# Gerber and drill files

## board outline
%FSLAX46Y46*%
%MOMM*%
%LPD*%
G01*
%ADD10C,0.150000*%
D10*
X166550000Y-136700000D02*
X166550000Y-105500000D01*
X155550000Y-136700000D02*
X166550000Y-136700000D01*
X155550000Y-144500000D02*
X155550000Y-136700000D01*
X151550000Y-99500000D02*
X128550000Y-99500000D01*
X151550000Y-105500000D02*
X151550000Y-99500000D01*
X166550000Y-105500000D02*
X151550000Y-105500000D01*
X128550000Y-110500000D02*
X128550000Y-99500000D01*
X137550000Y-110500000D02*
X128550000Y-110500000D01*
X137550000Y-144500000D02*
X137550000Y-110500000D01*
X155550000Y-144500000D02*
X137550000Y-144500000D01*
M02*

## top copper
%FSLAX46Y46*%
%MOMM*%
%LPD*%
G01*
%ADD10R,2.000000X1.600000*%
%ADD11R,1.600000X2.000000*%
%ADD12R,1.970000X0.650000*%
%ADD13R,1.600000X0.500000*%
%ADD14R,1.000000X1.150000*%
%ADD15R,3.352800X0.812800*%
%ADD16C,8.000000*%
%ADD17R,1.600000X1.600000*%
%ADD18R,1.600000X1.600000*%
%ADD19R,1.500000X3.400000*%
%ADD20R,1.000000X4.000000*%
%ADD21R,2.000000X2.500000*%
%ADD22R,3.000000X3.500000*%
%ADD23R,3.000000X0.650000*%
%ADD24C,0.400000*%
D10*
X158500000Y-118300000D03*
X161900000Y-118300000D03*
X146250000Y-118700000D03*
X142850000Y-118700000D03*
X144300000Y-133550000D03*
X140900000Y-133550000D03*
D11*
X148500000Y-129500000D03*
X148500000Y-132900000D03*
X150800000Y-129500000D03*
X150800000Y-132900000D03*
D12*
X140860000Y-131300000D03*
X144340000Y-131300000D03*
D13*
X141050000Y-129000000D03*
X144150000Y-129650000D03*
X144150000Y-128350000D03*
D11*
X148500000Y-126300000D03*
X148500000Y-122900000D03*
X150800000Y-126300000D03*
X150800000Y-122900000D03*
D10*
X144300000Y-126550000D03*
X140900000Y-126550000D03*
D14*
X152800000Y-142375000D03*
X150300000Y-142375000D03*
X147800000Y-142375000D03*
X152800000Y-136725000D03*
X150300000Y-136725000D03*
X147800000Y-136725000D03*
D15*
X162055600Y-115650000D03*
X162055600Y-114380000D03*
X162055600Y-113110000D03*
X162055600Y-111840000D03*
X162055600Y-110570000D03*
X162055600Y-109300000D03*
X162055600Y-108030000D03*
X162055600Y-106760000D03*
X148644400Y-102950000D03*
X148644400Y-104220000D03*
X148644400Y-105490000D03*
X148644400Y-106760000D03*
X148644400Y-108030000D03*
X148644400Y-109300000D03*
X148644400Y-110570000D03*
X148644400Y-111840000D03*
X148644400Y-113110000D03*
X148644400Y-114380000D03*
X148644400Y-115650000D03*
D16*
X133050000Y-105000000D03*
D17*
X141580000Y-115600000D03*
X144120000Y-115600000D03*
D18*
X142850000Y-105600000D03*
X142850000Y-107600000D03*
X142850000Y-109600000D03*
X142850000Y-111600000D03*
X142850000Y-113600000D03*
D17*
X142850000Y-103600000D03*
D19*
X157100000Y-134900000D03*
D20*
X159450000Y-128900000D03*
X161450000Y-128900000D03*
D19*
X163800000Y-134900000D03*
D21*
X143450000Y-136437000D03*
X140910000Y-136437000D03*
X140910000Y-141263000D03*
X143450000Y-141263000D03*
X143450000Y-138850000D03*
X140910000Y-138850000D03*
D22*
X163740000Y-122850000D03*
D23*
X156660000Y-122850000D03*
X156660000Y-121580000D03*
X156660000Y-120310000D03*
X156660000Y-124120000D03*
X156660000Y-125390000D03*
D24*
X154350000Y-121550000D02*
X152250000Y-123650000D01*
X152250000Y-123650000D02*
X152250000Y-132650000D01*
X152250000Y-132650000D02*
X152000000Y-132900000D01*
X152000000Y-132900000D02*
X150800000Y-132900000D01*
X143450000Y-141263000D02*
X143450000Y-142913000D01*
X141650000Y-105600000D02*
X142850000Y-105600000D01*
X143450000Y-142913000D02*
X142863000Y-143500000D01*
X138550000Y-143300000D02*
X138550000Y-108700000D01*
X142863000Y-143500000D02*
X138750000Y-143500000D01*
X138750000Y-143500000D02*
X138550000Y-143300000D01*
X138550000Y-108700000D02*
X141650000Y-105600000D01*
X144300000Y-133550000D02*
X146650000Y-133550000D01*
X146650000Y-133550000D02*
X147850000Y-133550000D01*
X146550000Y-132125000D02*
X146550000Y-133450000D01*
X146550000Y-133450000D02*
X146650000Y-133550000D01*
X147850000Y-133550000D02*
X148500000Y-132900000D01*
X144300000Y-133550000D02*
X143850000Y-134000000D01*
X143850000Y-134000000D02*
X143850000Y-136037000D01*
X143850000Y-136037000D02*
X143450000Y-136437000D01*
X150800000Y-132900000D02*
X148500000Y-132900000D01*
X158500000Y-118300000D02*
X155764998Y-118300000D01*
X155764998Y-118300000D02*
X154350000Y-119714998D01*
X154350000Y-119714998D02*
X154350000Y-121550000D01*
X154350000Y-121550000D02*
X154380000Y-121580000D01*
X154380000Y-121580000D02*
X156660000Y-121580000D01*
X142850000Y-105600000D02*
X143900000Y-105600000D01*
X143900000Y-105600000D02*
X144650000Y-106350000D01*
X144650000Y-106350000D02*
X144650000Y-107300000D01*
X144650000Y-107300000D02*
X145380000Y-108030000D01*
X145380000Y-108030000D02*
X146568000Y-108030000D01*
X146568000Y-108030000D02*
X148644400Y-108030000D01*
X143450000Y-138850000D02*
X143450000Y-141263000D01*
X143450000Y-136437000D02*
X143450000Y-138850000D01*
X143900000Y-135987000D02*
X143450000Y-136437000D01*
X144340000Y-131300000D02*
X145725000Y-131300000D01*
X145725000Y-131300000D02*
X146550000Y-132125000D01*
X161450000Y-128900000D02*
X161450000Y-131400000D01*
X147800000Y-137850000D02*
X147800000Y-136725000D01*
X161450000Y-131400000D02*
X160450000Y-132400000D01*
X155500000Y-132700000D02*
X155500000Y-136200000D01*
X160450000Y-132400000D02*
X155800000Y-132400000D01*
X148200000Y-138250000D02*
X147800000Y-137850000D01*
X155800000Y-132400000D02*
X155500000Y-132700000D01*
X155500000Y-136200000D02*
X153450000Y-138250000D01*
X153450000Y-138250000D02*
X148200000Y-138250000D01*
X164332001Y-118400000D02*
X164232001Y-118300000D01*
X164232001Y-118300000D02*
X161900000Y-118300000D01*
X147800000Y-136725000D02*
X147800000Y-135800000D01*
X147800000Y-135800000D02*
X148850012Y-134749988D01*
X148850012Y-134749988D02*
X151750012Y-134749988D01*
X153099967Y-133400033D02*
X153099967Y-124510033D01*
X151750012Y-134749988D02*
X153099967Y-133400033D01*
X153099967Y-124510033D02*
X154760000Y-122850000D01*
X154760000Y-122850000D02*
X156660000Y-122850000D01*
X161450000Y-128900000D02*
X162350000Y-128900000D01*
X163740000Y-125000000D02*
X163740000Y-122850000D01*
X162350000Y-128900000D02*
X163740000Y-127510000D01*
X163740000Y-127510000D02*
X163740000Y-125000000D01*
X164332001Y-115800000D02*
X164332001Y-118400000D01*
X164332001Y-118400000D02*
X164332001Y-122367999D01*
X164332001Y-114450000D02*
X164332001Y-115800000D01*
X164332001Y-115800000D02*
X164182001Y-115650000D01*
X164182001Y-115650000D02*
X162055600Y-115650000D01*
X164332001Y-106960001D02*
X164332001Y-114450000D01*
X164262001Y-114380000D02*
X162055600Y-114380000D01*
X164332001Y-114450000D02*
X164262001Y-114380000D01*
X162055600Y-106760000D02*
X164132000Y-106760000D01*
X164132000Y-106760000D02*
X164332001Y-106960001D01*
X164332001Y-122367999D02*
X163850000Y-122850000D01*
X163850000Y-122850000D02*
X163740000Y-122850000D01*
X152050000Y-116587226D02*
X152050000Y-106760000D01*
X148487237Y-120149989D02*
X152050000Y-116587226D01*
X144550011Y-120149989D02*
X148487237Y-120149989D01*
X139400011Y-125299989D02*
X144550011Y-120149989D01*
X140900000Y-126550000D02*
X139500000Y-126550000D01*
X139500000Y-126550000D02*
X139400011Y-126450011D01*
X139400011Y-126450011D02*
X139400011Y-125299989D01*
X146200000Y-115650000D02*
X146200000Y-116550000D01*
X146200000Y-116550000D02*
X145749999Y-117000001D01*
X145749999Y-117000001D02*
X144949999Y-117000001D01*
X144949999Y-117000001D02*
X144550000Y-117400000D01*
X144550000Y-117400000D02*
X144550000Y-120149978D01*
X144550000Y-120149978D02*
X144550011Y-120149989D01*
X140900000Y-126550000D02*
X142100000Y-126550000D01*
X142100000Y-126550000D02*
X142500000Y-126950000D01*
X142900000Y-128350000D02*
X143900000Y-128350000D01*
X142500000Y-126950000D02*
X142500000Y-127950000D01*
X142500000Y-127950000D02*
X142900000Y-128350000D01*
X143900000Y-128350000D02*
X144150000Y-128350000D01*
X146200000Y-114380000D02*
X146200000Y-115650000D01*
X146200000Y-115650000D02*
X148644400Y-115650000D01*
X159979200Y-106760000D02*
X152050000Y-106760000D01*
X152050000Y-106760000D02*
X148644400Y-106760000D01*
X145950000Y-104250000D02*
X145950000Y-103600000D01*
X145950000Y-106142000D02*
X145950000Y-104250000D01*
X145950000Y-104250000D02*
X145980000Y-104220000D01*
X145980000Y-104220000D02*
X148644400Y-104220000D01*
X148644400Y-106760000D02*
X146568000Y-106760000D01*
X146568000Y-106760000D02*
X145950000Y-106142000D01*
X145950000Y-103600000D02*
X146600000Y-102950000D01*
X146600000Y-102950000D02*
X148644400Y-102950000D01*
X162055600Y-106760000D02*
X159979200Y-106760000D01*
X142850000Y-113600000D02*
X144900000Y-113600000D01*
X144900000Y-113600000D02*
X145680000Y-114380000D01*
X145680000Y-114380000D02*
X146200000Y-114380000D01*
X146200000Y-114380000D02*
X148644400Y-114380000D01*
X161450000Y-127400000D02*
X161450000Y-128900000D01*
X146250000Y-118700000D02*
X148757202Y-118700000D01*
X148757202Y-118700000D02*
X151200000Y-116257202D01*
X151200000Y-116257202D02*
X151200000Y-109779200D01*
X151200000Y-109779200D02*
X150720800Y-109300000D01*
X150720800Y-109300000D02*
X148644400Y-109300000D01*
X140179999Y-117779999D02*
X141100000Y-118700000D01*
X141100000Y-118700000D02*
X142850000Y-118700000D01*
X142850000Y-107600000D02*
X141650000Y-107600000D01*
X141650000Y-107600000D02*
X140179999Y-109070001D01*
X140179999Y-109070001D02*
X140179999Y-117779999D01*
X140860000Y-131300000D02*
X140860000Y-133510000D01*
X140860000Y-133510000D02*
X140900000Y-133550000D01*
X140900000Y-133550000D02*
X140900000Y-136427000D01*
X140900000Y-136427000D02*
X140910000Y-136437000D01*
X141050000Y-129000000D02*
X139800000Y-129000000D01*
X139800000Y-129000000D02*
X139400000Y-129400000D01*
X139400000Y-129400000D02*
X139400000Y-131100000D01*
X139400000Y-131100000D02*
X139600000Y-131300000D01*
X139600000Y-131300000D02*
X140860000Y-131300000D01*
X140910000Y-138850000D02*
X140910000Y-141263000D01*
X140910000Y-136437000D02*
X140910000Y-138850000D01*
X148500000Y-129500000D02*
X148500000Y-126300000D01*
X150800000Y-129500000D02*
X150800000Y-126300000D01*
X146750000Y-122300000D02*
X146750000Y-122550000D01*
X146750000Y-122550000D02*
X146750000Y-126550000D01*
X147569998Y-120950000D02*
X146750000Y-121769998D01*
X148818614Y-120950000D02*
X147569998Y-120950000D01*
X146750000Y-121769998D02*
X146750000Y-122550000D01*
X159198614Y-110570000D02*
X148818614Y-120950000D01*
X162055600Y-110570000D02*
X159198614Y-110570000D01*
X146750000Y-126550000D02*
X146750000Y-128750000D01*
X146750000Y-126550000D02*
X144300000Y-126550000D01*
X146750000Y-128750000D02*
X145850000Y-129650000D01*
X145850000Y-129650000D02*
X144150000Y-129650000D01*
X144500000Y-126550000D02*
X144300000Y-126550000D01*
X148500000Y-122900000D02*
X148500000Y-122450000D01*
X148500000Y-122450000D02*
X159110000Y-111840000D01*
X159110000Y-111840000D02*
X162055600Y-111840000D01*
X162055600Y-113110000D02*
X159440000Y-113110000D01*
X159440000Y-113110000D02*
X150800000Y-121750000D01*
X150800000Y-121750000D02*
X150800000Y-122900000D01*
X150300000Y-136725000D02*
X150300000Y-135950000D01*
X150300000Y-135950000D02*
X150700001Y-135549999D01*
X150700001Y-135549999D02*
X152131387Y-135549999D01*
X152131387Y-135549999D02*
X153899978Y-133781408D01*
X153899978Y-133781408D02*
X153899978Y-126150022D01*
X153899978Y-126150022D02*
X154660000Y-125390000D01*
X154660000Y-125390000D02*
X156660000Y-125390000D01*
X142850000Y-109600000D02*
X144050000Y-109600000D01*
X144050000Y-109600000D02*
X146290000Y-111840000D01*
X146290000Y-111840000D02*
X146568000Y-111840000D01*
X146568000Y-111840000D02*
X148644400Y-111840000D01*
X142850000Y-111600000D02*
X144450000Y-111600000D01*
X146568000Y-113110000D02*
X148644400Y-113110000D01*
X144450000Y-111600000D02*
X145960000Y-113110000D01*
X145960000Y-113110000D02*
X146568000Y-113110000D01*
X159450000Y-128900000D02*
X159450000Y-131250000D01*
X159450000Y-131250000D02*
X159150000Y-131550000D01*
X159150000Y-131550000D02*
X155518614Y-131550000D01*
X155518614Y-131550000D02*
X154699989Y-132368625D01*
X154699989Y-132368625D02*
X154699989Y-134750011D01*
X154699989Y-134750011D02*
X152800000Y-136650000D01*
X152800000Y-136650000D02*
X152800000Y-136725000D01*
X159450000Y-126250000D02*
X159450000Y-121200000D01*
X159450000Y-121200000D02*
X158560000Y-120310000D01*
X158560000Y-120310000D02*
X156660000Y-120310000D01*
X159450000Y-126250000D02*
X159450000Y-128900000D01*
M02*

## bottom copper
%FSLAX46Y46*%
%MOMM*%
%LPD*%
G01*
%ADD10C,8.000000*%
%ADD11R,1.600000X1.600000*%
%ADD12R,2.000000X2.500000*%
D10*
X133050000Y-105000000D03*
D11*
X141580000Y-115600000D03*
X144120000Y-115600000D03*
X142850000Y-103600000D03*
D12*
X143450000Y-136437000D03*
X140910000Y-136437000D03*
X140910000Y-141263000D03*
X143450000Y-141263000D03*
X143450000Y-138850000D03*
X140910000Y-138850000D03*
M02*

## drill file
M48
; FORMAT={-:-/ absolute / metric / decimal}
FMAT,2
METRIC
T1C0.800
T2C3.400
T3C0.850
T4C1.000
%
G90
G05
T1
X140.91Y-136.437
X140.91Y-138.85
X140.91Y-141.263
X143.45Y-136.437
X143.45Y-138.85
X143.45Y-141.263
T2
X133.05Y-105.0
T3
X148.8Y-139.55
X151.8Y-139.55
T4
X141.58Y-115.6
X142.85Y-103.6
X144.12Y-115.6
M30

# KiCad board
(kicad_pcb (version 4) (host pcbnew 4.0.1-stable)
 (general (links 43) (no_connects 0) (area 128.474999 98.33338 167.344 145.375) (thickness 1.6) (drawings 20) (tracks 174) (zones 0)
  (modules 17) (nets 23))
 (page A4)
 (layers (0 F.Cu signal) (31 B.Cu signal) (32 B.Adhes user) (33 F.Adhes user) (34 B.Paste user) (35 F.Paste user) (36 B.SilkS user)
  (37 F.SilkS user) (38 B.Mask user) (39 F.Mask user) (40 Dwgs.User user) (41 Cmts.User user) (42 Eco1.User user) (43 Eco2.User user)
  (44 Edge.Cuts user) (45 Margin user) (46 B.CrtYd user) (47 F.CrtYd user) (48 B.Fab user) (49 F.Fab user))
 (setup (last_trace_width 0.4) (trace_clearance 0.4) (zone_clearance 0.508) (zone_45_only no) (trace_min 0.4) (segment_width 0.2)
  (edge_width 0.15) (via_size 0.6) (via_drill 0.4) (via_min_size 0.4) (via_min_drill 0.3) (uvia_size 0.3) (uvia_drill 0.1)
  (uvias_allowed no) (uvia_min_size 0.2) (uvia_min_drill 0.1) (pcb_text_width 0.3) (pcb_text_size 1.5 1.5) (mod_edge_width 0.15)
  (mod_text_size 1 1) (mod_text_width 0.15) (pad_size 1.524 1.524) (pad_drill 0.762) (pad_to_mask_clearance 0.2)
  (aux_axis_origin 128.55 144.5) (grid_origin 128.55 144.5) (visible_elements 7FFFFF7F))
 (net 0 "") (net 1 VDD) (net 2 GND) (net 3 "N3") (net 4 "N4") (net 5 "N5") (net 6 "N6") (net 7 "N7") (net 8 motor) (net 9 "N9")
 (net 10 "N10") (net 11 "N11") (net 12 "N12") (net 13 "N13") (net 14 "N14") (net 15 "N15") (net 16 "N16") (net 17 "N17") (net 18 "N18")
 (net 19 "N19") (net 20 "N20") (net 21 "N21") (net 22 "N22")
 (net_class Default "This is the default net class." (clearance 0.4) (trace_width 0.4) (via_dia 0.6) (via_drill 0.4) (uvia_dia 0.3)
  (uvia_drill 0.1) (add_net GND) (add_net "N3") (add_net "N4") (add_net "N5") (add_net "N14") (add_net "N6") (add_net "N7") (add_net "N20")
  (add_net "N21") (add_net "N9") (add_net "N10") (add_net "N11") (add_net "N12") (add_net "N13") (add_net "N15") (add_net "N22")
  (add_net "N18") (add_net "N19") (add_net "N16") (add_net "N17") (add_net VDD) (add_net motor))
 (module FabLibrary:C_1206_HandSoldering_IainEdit (layer F.Cu) (at 160.2 118.3)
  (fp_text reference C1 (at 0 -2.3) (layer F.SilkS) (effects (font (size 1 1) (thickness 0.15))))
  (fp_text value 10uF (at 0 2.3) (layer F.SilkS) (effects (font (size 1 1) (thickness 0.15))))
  (pad 1 smd rect (at -1.7 0) (size 2 1.6) (layers F.Cu F.Paste F.Mask) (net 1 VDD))
  (pad 2 smd rect (at 1.7 0) (size 2 1.6) (layers F.Cu F.Paste F.Mask) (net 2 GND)))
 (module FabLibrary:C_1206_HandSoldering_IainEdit (layer F.Cu) (at 144.55 118.7 180)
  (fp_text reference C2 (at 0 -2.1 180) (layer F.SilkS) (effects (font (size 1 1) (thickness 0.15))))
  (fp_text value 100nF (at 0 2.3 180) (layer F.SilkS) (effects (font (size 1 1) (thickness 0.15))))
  (pad 1 smd rect (at -1.7 0 180) (size 2 1.6) (layers F.Cu F.Paste F.Mask) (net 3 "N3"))
  (pad 2 smd rect (at 1.7 0 180) (size 2 1.6) (layers F.Cu F.Paste F.Mask) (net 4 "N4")))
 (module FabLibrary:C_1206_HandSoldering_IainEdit (layer F.Cu) (at 142.6 133.55 180)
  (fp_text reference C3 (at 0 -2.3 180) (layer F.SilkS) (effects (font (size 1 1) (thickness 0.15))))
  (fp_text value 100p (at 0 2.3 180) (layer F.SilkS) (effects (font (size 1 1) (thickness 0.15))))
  (pad 1 smd rect (at -1.7 0 180) (size 2 1.6) (layers F.Cu F.Paste F.Mask) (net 1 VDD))
  (pad 2 smd rect (at 1.7 0 180) (size 2 1.6) (layers F.Cu F.Paste F.Mask) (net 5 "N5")))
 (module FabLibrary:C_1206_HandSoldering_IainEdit (layer F.Cu) (at 148.5 131.2 270)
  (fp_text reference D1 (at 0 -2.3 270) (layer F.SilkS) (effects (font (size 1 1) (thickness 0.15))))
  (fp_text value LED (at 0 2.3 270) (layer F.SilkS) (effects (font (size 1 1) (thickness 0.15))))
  (pad 1 smd rect (at -1.7 0 270) (size 2 1.6) (layers F.Cu F.Paste F.Mask) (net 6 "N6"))
  (pad 2 smd rect (at 1.7 0 270) (size 2 1.6) (layers F.Cu F.Paste F.Mask) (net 1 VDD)))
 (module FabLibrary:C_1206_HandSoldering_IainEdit (layer F.Cu) (at 150.8 131.2 270)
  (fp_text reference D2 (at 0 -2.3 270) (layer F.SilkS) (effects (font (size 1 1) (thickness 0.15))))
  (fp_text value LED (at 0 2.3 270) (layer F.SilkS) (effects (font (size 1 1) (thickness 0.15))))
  (pad 1 smd rect (at -1.7 0 270) (size 2 1.6) (layers F.Cu F.Paste F.Mask) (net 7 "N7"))
  (pad 2 smd rect (at 1.7 0 270) (size 2 1.6) (layers F.Cu F.Paste F.Mask) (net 1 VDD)))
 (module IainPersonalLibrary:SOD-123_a (layer F.Cu) (at 142.6 131.3 180)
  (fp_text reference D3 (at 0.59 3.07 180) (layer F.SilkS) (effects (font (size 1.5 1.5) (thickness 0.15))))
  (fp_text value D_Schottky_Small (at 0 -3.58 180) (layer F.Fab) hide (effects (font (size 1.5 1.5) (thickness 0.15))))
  (pad 2 smd rect (at 1.74 0 180) (size 1.97 0.65) (layers F.Cu F.Paste F.Mask) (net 5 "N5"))
  (pad 1 smd rect (at -1.74 0 180) (size 1.97 0.65) (layers F.Cu F.Paste F.Mask) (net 1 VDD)))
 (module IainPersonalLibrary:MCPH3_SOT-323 (layer F.Cu) (at 142.6 129 90)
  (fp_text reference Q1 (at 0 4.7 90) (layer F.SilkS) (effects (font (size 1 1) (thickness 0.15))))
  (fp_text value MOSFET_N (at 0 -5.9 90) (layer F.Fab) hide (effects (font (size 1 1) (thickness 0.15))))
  (pad D smd rect (at 0 -1.55 90) (size 0.5 1.6) (layers F.Cu F.Paste F.Mask) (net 5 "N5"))
  (pad G smd rect (at -0.65 1.55 90) (size 0.5 1.6) (layers F.Cu F.Paste F.Mask) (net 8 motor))
  (pad S smd rect (at 0.65 1.55 90) (size 0.5 1.6) (layers F.Cu F.Paste F.Mask) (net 2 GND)))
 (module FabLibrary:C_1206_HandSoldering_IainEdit (layer F.Cu) (at 148.5 124.6 90)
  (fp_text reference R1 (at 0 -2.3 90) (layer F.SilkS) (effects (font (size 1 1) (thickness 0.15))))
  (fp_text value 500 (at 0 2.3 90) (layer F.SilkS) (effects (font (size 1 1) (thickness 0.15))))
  (pad 1 smd rect (at -1.7 0 90) (size 2 1.6) (layers F.Cu F.Paste F.Mask) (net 6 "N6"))
  (pad 2 smd rect (at 1.7 0 90) (size 2 1.6) (layers F.Cu F.Paste F.Mask) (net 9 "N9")))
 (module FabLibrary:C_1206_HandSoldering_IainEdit (layer F.Cu) (at 150.8 124.6 90)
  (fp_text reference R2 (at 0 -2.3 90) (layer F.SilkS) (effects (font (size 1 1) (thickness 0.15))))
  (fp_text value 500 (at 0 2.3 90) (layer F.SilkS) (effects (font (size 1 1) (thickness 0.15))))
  (pad 1 smd rect (at -1.7 0 90) (size 2 1.6) (layers F.Cu F.Paste F.Mask) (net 7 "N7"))
  (pad 2 smd rect (at 1.7 0 90) (size 2 1.6) (layers F.Cu F.Paste F.Mask) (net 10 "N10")))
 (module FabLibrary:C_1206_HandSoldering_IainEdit (layer F.Cu) (at 142.6 126.55 180)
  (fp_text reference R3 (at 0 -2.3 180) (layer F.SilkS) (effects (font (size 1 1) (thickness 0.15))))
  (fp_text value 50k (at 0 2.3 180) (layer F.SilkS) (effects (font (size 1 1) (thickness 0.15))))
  (pad 1 smd rect (at -1.7 0 180) (size 2 1.6) (layers F.Cu F.Paste F.Mask) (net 8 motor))
  (pad 2 smd rect (at 1.7 0 180) (size 2 1.6) (layers F.Cu F.Paste F.Mask) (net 2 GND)))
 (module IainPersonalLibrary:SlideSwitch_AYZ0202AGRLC (layer F.Cu) (at 150.3 139.55 180)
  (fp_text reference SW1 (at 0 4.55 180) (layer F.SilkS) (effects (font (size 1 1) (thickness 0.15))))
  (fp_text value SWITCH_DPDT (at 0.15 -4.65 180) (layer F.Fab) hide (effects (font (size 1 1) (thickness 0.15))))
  (pad "" np_thru_hole circle (at 1.5 0 180) (size 0.85 0.85) (drill 0.85) (layers *.Cu *.Mask))
  (pad "" np_thru_hole circle (at -1.5 0 180) (size 0.85 0.85) (drill 0.85) (layers *.Cu *.Mask))
  (pad 1 smd rect (at -2.5 -2.825 180) (size 1 1.15) (layers F.Cu F.Paste F.Mask) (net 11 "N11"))
  (pad 2 smd rect (at 0 -2.825 180) (size 1 1.15) (layers F.Cu F.Paste F.Mask) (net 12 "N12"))
  (pad 3 smd rect (at 2.5 -2.825 180) (size 1 1.15) (layers F.Cu F.Paste F.Mask) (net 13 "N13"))
  (pad 4 smd rect (at -2.5 2.825 180) (size 1 1.15) (layers F.Cu F.Paste F.Mask) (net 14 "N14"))
  (pad 5 smd rect (at 0 2.825 180) (size 1 1.15) (layers F.Cu F.Paste F.Mask) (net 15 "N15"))
  (pad 6 smd rect (at 2.5 2.825 180) (size 1 1.15) (layers F.Cu F.Paste F.Mask) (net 2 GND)))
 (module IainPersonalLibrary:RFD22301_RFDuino (layer F.Cu) (at 155.35 109.3 180) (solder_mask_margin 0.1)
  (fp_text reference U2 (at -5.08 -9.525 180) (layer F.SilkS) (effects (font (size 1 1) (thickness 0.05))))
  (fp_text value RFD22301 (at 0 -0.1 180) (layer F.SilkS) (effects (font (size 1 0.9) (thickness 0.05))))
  (pad P$1 smd rect (at -6.7056 -6.35 180) (size 3.3528 0.8128) (layers F.Cu F.Paste F.Mask) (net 2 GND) (solder_mask_margin 0.2))
  (pad P$2 smd rect (at -6.7056 -5.08 180) (size 3.3528 0.8128) (layers F.Cu F.Paste F.Mask) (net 2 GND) (solder_mask_margin 0.2))
  (pad P$3 smd rect (at -6.7056 -3.81 180) (size 3.3528 0.8128) (layers F.Cu F.Paste F.Mask) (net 10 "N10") (solder_mask_margin 0.2))
  (pad P$4 smd rect (at -6.7056 -2.54 180) (size 3.3528 0.8128) (layers F.Cu F.Paste F.Mask) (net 9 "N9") (solder_mask_margin 0.2))
  (pad P$5 smd rect (at -6.7056 -1.27 180) (size 3.3528 0.8128) (layers F.Cu F.Paste F.Mask) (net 8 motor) (solder_mask_margin 0.2))
  (pad P$6 smd rect (at -6.7056 0 180) (size 3.3528 0.8128) (layers F.Cu F.Paste F.Mask) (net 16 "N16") (solder_mask_margin 0.2))
  (pad P$7 smd rect (at -6.7056 1.27 180) (size 3.3528 0.8128) (layers F.Cu F.Paste F.Mask) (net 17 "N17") (solder_mask_margin 0.2))
  (pad P$8 smd rect (at -6.7056 2.54 180) (size 3.3528 0.8128) (layers F.Cu F.Paste F.Mask) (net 2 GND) (solder_mask_margin 0.2))
  (pad P$9 smd rect (at 6.7056 6.35 180) (size 3.3528 0.8128) (layers F.Cu F.Paste F.Mask) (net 2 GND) (solder_mask_margin 0.2))
  (pad P$10 smd rect (at 6.7056 5.08 180) (size 3.3528 0.8128) (layers F.Cu F.Paste F.Mask) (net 2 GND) (solder_mask_margin 0.2))
  (pad P$11 smd rect (at 6.7056 3.81 180) (size 3.3528 0.8128) (layers F.Cu F.Paste F.Mask) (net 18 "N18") (solder_mask_margin 0.2))
  (pad P$12 smd rect (at 6.7056 2.54 180) (size 3.3528 0.8128) (layers F.Cu F.Paste F.Mask) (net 2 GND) (solder_mask_margin 0.2))
  (pad P$13 smd rect (at 6.7056 1.27 180) (size 3.3528 0.8128) (layers F.Cu F.Paste F.Mask) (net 1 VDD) (solder_mask_margin 0.2))
  (pad P$14 smd rect (at 6.7056 0 180) (size 3.3528 0.8128) (layers F.Cu F.Paste F.Mask) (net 3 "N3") (solder_mask_margin 0.2))
  (pad P$15 smd rect (at 6.7056 -1.27 180) (size 3.3528 0.8128) (layers F.Cu F.Paste F.Mask) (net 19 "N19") (solder_mask_margin 0.2))
  (pad P$16 smd rect (at 6.7056 -2.54 180) (size 3.3528 0.8128) (layers F.Cu F.Paste F.Mask) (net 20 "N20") (solder_mask_margin 0.2))
  (pad P$17 smd rect (at 6.7056 -3.81 180) (size 3.3528 0.8128) (layers F.Cu F.Paste F.Mask) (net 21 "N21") (solder_mask_margin 0.2))
  (pad P$18 smd rect (at 6.7056 -5.08 180) (size 3.3528 0.8128) (layers F.Cu F.Paste F.Mask) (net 2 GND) (solder_mask_margin 0.2))
  (pad P$19 smd rect (at 6.7056 -6.35 180) (size 3.3528 0.8128) (layers F.Cu F.Paste F.Mask) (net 2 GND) (solder_mask_margin 0.2)))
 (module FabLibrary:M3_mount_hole (layer F.Cu) (at 133.05 105)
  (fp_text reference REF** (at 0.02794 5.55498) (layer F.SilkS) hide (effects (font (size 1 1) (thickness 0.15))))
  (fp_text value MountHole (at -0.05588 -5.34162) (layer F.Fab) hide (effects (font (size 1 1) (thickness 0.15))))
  (pad 1 thru_hole circle (at 0 0) (size 8 8) (drill 3.4) (layers *.Cu *.Mask F.SilkS)))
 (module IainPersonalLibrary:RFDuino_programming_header (layer F.Cu) (at 142.85 109.6 270)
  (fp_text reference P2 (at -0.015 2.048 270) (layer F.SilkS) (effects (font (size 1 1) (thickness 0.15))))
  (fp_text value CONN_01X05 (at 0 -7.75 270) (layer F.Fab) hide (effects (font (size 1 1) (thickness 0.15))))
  (pad "" np_thru_hole rect (at 6 1.27 270) (size 1.6 1.6) (drill 1) (layers *.Cu *.Mask F.SilkS))
  (pad "" np_thru_hole rect (at 6 -1.27 270) (size 1.6 1.6) (drill 1) (layers *.Cu *.Mask F.SilkS))
  (pad 1 smd rect (at -4 0 270) (size 1.6 1.6) (layers F.Cu F.Paste F.Mask) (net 1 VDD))
  (pad 2 smd rect (at -2 0 270) (size 1.6 1.6) (layers F.Cu F.Paste F.Mask) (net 4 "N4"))
  (pad 3 smd rect (at 0 0 270) (size 1.6 1.6) (layers F.Cu F.Paste F.Mask) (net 20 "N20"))
  (pad 4 smd rect (at 2 0 270) (size 1.6 1.6) (layers F.Cu F.Paste F.Mask) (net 21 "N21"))
  (pad 5 smd rect (at 4 0 270) (size 1.6 1.6) (layers F.Cu F.Paste F.Mask) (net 2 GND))
  (pad "" np_thru_hole rect (at -6 0 270) (size 1.6 1.6) (drill 1) (layers *.Cu *.Mask F.SilkS)))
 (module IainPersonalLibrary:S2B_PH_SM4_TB (layer F.Cu) (at 160.45 129.15 180)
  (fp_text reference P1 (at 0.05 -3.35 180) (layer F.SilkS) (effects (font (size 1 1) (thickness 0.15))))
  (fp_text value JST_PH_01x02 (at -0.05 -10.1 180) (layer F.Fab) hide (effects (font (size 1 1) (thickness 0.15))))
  (pad x smd rect (at 3.35 -5.75 180) (size 1.5 3.4) (layers F.Cu F.Paste F.Mask))
  (pad 1 smd rect (at 1 0.25 180) (size 1 4) (layers F.Cu F.Paste F.Mask) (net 14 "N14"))
  (pad 2 smd rect (at -1 0.25 180) (size 1 4) (layers F.Cu F.Paste F.Mask) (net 2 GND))
  (pad x smd rect (at -3.35 -5.75 180) (size 1.5 3.4) (layers F.Cu F.Paste F.Mask)))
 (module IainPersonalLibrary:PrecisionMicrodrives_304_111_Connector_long (layer F.Cu) (at 143.45 138.85 180)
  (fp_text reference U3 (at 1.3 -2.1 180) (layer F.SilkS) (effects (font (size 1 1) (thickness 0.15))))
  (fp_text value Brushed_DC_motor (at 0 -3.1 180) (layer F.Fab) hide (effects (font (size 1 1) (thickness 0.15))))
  (pad 1 thru_hole rect (at 0 2.413 180) (size 2 2.5) (drill 0.8) (layers *.Mask F.Cu F.SilkS) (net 1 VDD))
  (pad 2 thru_hole rect (at 2.54 2.413 180) (size 2 2.5) (drill 0.8) (layers *.Mask F.Cu F.SilkS) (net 5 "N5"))
  (pad 2 thru_hole rect (at 2.54 -2.413 180) (size 2 2.5) (drill 0.8) (layers *.Mask F.Cu F.SilkS) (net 5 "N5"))
  (pad 1 thru_hole rect (at 0 -2.413 180) (size 2 2.5) (drill 0.8) (layers *.Mask F.Cu F.SilkS) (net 1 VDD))
  (pad 1 thru_hole rect (at 0 0 180) (size 2 2.5) (drill 0.8) (layers *.Mask F.Cu F.SilkS) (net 1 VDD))
  (pad 2 thru_hole rect (at 2.54 0 180) (size 2 2.5) (drill 0.8) (layers *.Mask F.Cu F.SilkS) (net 5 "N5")))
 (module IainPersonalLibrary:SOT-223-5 (layer F.Cu) (at 160.2 122.85 270)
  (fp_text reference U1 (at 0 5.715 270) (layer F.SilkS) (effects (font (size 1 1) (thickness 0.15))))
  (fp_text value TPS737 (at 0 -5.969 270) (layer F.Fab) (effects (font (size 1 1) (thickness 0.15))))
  (pad 3 smd rect (at 0 -3.54 270) (size 3.5 3) (layers F.Cu F.Paste F.Mask) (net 2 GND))
  (pad 3 smd rect (at 0 3.54 270) (size 0.65 3) (layers F.Cu F.Paste F.Mask) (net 2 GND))
  (pad 2 smd rect (at -1.27 3.54 270) (size 0.65 3) (layers F.Cu F.Paste F.Mask) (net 1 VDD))
  (pad 1 smd rect (at -2.54 3.54 270) (size 0.65 3) (layers F.Cu F.Paste F.Mask) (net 14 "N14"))
  (pad 4 smd rect (at 1.27 3.54 270) (size 0.65 3) (layers F.Cu F.Paste F.Mask) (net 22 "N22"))
  (pad 5 smd rect (at 2.54 3.54 270) (size 0.65 3) (layers F.Cu F.Paste F.Mask) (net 15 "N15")))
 (gr_line (start 166.55 136.7) (end 166.55 105.5) (angle 90) (layer Edge.Cuts) (width 0.15))
 (gr_line (start 155.55 136.7) (end 166.55 136.7) (angle 90) (layer Edge.Cuts) (width 0.15))
 (gr_line (start 155.55 144.5) (end 155.55 136.7) (angle 90) (layer Edge.Cuts) (width 0.15))
 (gr_line (start 151.55 99.5) (end 128.55 99.5) (angle 90) (layer Edge.Cuts) (width 0.15))
 (gr_line (start 151.55 105.5) (end 151.55 99.5) (angle 90) (layer Edge.Cuts) (width 0.15))
 (gr_line (start 166.55 105.5) (end 151.55 105.5) (angle 90) (layer Edge.Cuts) (width 0.15))
 (gr_line (start 128.55 110.5) (end 128.55 99.5) (angle 90) (layer Edge.Cuts) (width 0.15))
 (gr_line (start 137.55 110.5) (end 128.55 110.5) (angle 90) (layer Edge.Cuts) (width 0.15))
 (gr_line (start 137.55 144.5) (end 137.55 110.5) (angle 90) (layer Edge.Cuts) (width 0.15))
 (gr_line (start 155.55 144.5) (end 137.55 144.5) (angle 90) (layer Edge.Cuts) (width 0.15))
 (segment (start 154.35 121.55) (end 152.25 123.65) (width 0.4) (layer F.Cu) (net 1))
 (segment (start 152.25 123.65) (end 152.25 132.65) (width 0.4) (layer F.Cu) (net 1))
 (segment (start 152.25 132.65) (end 152 132.9) (width 0.4) (layer F.Cu) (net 1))
 (segment (start 152 132.9) (end 150.8 132.9) (width 0.4) (layer F.Cu) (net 1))
 (segment (start 143.45 141.263) (end 143.45 142.913) (width 0.4) (layer F.Cu) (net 1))
 (segment (start 141.65 105.6) (end 142.85 105.6) (width 0.4) (layer F.Cu) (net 1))
 (segment (start 143.45 142.913) (end 142.863 143.5) (width 0.4) (layer F.Cu) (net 1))
 (segment (start 138.55 143.3) (end 138.55 108.7) (width 0.4) (layer F.Cu) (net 1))
 (segment (start 142.863 143.5) (end 138.75 143.5) (width 0.4) (layer F.Cu) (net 1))
 (segment (start 138.75 143.5) (end 138.55 143.3) (width 0.4) (layer F.Cu) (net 1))
 (segment (start 138.55 108.7) (end 141.65 105.6) (width 0.4) (layer F.Cu) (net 1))
 (segment (start 144.3 133.55) (end 146.65 133.55) (width 0.4) (layer F.Cu) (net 1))
 (segment (start 146.65 133.55) (end 147.85 133.55) (width 0.4) (layer F.Cu) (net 1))
 (segment (start 146.55 132.125) (end 146.55 133.45) (width 0.4) (layer F.Cu) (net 1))
 (segment (start 146.55 133.45) (end 146.65 133.55) (width 0.4) (layer F.Cu) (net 1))
 (segment (start 147.85 133.55) (end 148.5 132.9) (width 0.4) (layer F.Cu) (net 1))
 (segment (start 144.3 133.55) (end 143.85 134) (width 0.4) (layer F.Cu) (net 1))
 (segment (start 143.85 134) (end 143.85 136.037) (width 0.4) (layer F.Cu) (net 1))
 (segment (start 143.85 136.037) (end 143.45 136.437) (width 0.4) (layer F.Cu) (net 1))
 (segment (start 150.8 132.9) (end 148.5 132.9) (width 0.4) (layer F.Cu) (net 1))
 (segment (start 158.5 118.3) (end 155.764998 118.3) (width 0.4) (layer F.Cu) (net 1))
 (segment (start 155.764998 118.3) (end 154.35 119.714998) (width 0.4) (layer F.Cu) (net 1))
 (segment (start 154.35 119.714998) (end 154.35 121.55) (width 0.4) (layer F.Cu) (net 1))
 (segment (start 154.35 121.55) (end 154.38 121.58) (width 0.4) (layer F.Cu) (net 1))
 (segment (start 154.38 121.58) (end 156.66 121.58) (width 0.4) (layer F.Cu) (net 1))
 (segment (start 142.85 105.6) (end 143.9 105.6) (width 0.4) (layer F.Cu) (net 1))
 (segment (start 143.9 105.6) (end 144.65 106.35) (width 0.4) (layer F.Cu) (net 1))
 (segment (start 144.65 106.35) (end 144.65 107.3) (width 0.4) (layer F.Cu) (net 1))
 (segment (start 144.65 107.3) (end 145.38 108.03) (width 0.4) (layer F.Cu) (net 1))
 (segment (start 145.38 108.03) (end 146.568 108.03) (width 0.4) (layer F.Cu) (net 1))
 (segment (start 146.568 108.03) (end 148.6444 108.03) (width 0.4) (layer F.Cu) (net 1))
 (segment (start 143.45 138.85) (end 143.45 141.263) (width 0.4) (layer F.Cu) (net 1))
 (segment (start 143.45 136.437) (end 143.45 138.85) (width 0.4) (layer F.Cu) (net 1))
 (segment (start 143.9 135.987) (end 143.45 136.437) (width 0.4) (layer F.Cu) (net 1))
 (segment (start 144.34 131.3) (end 145.725 131.3) (width 0.4) (layer F.Cu) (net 1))
 (segment (start 145.725 131.3) (end 146.55 132.125) (width 0.4) (layer F.Cu) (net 1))
 (segment (start 161.45 128.9) (end 161.45 131.4) (width 0.4) (layer F.Cu) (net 2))
 (segment (start 147.8 137.85) (end 147.8 136.725) (width 0.4) (layer F.Cu) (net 2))
 (segment (start 161.45 131.4) (end 160.45 132.4) (width 0.4) (layer F.Cu) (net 2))
 (segment (start 155.5 132.7) (end 155.5 136.2) (width 0.4) (layer F.Cu) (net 2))
 (segment (start 160.45 132.4) (end 155.8 132.4) (width 0.4) (layer F.Cu) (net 2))
 (segment (start 148.2 138.25) (end 147.8 137.85) (width 0.4) (layer F.Cu) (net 2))
 (segment (start 155.8 132.4) (end 155.5 132.7) (width 0.4) (layer F.Cu) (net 2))
 (segment (start 155.5 136.2) (end 153.45 138.25) (width 0.4) (layer F.Cu) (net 2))
 (segment (start 153.45 138.25) (end 148.2 138.25) (width 0.4) (layer F.Cu) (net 2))
 (segment (start 164.332001 118.4) (end 164.232001 118.3) (width 0.4) (layer F.Cu) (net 2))
 (segment (start 164.232001 118.3) (end 161.9 118.3) (width 0.4) (layer F.Cu) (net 2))
 (segment (start 147.8 136.725) (end 147.8 135.8) (width 0.4) (layer F.Cu) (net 2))
 (segment (start 147.8 135.8) (end 148.850012 134.749988) (width 0.4) (layer F.Cu) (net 2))
 (segment (start 148.850012 134.749988) (end 151.750012 134.749988) (width 0.4) (layer F.Cu) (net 2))
 (segment (start 153.099967 133.400033) (end 153.099967 124.510033) (width 0.4) (layer F.Cu) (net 2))
 (segment (start 151.750012 134.749988) (end 153.099967 133.400033) (width 0.4) (layer F.Cu) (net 2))
 (segment (start 153.099967 124.510033) (end 154.76 122.85) (width 0.4) (layer F.Cu) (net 2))
 (segment (start 154.76 122.85) (end 156.66 122.85) (width 0.4) (layer F.Cu) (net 2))
 (segment (start 161.45 128.9) (end 162.35 128.9) (width 0.4) (layer F.Cu) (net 2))
 (segment (start 163.74 125) (end 163.74 122.85) (width 0.4) (layer F.Cu) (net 2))
 (segment (start 162.35 128.9) (end 163.74 127.51) (width 0.4) (layer F.Cu) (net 2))
 (segment (start 163.74 127.51) (end 163.74 125) (width 0.4) (layer F.Cu) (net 2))
 (segment (start 164.332001 115.8) (end 164.332001 118.4) (width 0.4) (layer F.Cu) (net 2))
 (segment (start 164.332001 118.4) (end 164.332001 122.367999) (width 0.4) (layer F.Cu) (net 2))
 (segment (start 164.332001 114.45) (end 164.332001 115.8) (width 0.4) (layer F.Cu) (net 2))
 (segment (start 164.332001 115.8) (end 164.182001 115.65) (width 0.4) (layer F.Cu) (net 2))
 (segment (start 164.182001 115.65) (end 162.0556 115.65) (width 0.4) (layer F.Cu) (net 2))
 (segment (start 164.332001 106.960001) (end 164.332001 114.45) (width 0.4) (layer F.Cu) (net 2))
 (segment (start 164.262001 114.38) (end 162.0556 114.38) (width 0.4) (layer F.Cu) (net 2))
 (segment (start 164.332001 114.45) (end 164.262001 114.38) (width 0.4) (layer F.Cu) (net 2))
 (segment (start 162.0556 106.76) (end 164.132 106.76) (width 0.4) (layer F.Cu) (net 2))
 (segment (start 164.132 106.76) (end 164.332001 106.960001) (width 0.4) (layer F.Cu) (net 2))
 (segment (start 164.332001 122.367999) (end 163.85 122.85) (width 0.4) (layer F.Cu) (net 2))
 (segment (start 163.85 122.85) (end 163.74 122.85) (width 0.4) (layer F.Cu) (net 2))
 (segment (start 152.05 116.587226) (end 152.05 106.76) (width 0.4) (layer F.Cu) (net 2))
 (segment (start 148.487237 120.149989) (end 152.05 116.587226) (width 0.4) (layer F.Cu) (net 2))
 (segment (start 144.550011 120.149989) (end 148.487237 120.149989) (width 0.4) (layer F.Cu) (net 2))
 (segment (start 139.400011 125.299989) (end 144.550011 120.149989) (width 0.4) (layer F.Cu) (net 2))
 (segment (start 140.9 126.55) (end 139.5 126.55) (width 0.4) (layer F.Cu) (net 2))
 (segment (start 139.5 126.55) (end 139.400011 126.450011) (width 0.4) (layer F.Cu) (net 2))
 (segment (start 139.400011 126.450011) (end 139.400011 125.299989) (width 0.4) (layer F.Cu) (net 2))
 (segment (start 146.2 115.65) (end 146.2 116.55) (width 0.4) (layer F.Cu) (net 2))
 (segment (start 146.2 116.55) (end 145.749999 117.000001) (width 0.4) (layer F.Cu) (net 2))
 (segment (start 145.749999 117.000001) (end 144.949999 117.000001) (width 0.4) (layer F.Cu) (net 2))
 (segment (start 144.949999 117.000001) (end 144.55 117.4) (width 0.4) (layer F.Cu) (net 2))
 (segment (start 144.55 117.4) (end 144.55 120.149978) (width 0.4) (layer F.Cu) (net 2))
 (segment (start 144.55 120.149978) (end 144.550011 120.149989) (width 0.4) (layer F.Cu) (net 2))
 (segment (start 140.9 126.55) (end 142.1 126.55) (width 0.4) (layer F.Cu) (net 2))
 (segment (start 142.1 126.55) (end 142.5 126.95) (width 0.4) (layer F.Cu) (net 2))
 (segment (start 142.9 128.35) (end 143.9 128.35) (width 0.4) (layer F.Cu) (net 2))
 (segment (start 142.5 126.95) (end 142.5 127.95) (width 0.4) (layer F.Cu) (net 2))
 (segment (start 142.5 127.95) (end 142.9 128.35) (width 0.4) (layer F.Cu) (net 2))
 (segment (start 143.9 128.35) (end 144.15 128.35) (width 0.4) (layer F.Cu) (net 2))
 (segment (start 146.2 114.38) (end 146.2 115.65) (width 0.4) (layer F.Cu) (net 2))
 (segment (start 146.2 115.65) (end 148.6444 115.65) (width 0.4) (layer F.Cu) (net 2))
 (segment (start 159.9792 106.76) (end 152.05 106.76) (width 0.4) (layer F.Cu) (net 2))
 (segment (start 152.05 106.76) (end 148.6444 106.76) (width 0.4) (layer F.Cu) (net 2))
 (segment (start 145.95 104.25) (end 145.95 103.6) (width 0.4) (layer F.Cu) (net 2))
 (segment (start 145.95 106.142) (end 145.95 104.25) (width 0.4) (layer F.Cu) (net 2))
 (segment (start 145.95 104.25) (end 145.98 104.22) (width 0.4) (layer F.Cu) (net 2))
 (segment (start 145.98 104.22) (end 148.6444 104.22) (width 0.4) (layer F.Cu) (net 2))
 (segment (start 148.6444 106.76) (end 146.568 106.76) (width 0.4) (layer F.Cu) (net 2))
 (segment (start 146.568 106.76) (end 145.95 106.142) (width 0.4) (layer F.Cu) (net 2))
 (segment (start 145.95 103.6) (end 146.6 102.95) (width 0.4) (layer F.Cu) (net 2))
 (segment (start 146.6 102.95) (end 148.6444 102.95) (width 0.4) (layer F.Cu) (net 2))
 (segment (start 162.0556 106.76) (end 159.9792 106.76) (width 0.4) (layer F.Cu) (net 2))
 (segment (start 142.85 113.6) (end 144.9 113.6) (width 0.4) (layer F.Cu) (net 2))
 (segment (start 144.9 113.6) (end 145.68 114.38) (width 0.4) (layer F.Cu) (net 2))
 (segment (start 145.68 114.38) (end 146.2 114.38) (width 0.4) (layer F.Cu) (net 2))
 (segment (start 146.2 114.38) (end 148.6444 114.38) (width 0.4) (layer F.Cu) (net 2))
 (segment (start 161.45 127.4) (end 161.45 128.9) (width 0.4) (layer F.Cu) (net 2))
 (segment (start 146.25 118.7) (end 148.757202 118.7) (width 0.4) (layer F.Cu) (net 3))
 (segment (start 148.757202 118.7) (end 151.2 116.257202) (width 0.4) (layer F.Cu) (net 3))
 (segment (start 151.2 116.257202) (end 151.2 109.7792) (width 0.4) (layer F.Cu) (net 3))
 (segment (start 151.2 109.7792) (end 150.7208 109.3) (width 0.4) (layer F.Cu) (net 3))
 (segment (start 150.7208 109.3) (end 148.6444 109.3) (width 0.4) (layer F.Cu) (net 3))
 (segment (start 140.179999 117.779999) (end 141.1 118.7) (width 0.4) (layer F.Cu) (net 4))
 (segment (start 141.1 118.7) (end 142.85 118.7) (width 0.4) (layer F.Cu) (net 4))
 (segment (start 142.85 107.6) (end 141.65 107.6) (width 0.4) (layer F.Cu) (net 4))
 (segment (start 141.65 107.6) (end 140.179999 109.070001) (width 0.4) (layer F.Cu) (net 4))
 (segment (start 140.179999 109.070001) (end 140.179999 117.779999) (width 0.4) (layer F.Cu) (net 4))
 (segment (start 140.86 131.3) (end 140.86 133.51) (width 0.4) (layer F.Cu) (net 5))
 (segment (start 140.86 133.51) (end 140.9 133.55) (width 0.4) (layer F.Cu) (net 5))
 (segment (start 140.9 133.55) (end 140.9 136.427) (width 0.4) (layer F.Cu) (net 5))
 (segment (start 140.9 136.427) (end 140.91 136.437) (width 0.4) (layer F.Cu) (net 5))
 (segment (start 141.05 129) (end 139.8 129) (width 0.4) (layer F.Cu) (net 5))
 (segment (start 139.8 129) (end 139.4 129.4) (width 0.4) (layer F.Cu) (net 5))
 (segment (start 139.4 129.4) (end 139.4 131.1) (width 0.4) (layer F.Cu) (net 5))
 (segment (start 139.4 131.1) (end 139.6 131.3) (width 0.4) (layer F.Cu) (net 5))
 (segment (start 139.6 131.3) (end 140.86 131.3) (width 0.4) (layer F.Cu) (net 5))
 (segment (start 140.91 138.85) (end 140.91 141.263) (width 0.4) (layer F.Cu) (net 5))
 (segment (start 140.91 136.437) (end 140.91 138.85) (width 0.4) (layer F.Cu) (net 5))
 (segment (start 148.5 129.5) (end 148.5 126.3) (width 0.4) (layer F.Cu) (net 6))
 (segment (start 150.8 129.5) (end 150.8 126.3) (width 0.4) (layer F.Cu) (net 7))
 (segment (start 146.75 122.3) (end 146.75 122.55) (width 0.4) (layer F.Cu) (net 8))
 (segment (start 146.75 122.55) (end 146.75 126.55) (width 0.4) (layer F.Cu) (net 8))
 (segment (start 147.569998 120.95) (end 146.75 121.769998) (width 0.4) (layer F.Cu) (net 8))
 (segment (start 148.818614 120.95) (end 147.569998 120.95) (width 0.4) (layer F.Cu) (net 8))
 (segment (start 146.75 121.769998) (end 146.75 122.55) (width 0.4) (layer F.Cu) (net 8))
 (segment (start 159.198614 110.57) (end 148.818614 120.95) (width 0.4) (layer F.Cu) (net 8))
 (segment (start 162.0556 110.57) (end 159.198614 110.57) (width 0.4) (layer F.Cu) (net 8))
 (segment (start 146.75 126.55) (end 146.75 128.75) (width 0.4) (layer F.Cu) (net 8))
 (segment (start 146.75 126.55) (end 144.3 126.55) (width 0.4) (layer F.Cu) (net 8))
 (segment (start 146.75 128.75) (end 145.85 129.65) (width 0.4) (layer F.Cu) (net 8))
 (segment (start 145.85 129.65) (end 144.15 129.65) (width 0.4) (layer F.Cu) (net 8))
 (segment (start 144.5 126.55) (end 144.3 126.55) (width 0.4) (layer F.Cu) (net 8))
 (segment (start 148.5 122.9) (end 148.5 122.45) (width 0.4) (layer F.Cu) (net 9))
 (segment (start 148.5 122.45) (end 159.11 111.84) (width 0.4) (layer F.Cu) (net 9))
 (segment (start 159.11 111.84) (end 162.0556 111.84) (width 0.4) (layer F.Cu) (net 9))
 (segment (start 162.0556 113.11) (end 159.44 113.11) (width 0.4) (layer F.Cu) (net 10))
 (segment (start 159.44 113.11) (end 150.8 121.75) (width 0.4) (layer F.Cu) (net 10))
 (segment (start 150.8 121.75) (end 150.8 122.9) (width 0.4) (layer F.Cu) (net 10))
 (segment (start 150.3 136.725) (end 150.3 135.95) (width 0.4) (layer F.Cu) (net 15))
 (segment (start 150.3 135.95) (end 150.700001 135.549999) (width 0.4) (layer F.Cu) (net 15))
 (segment (start 150.700001 135.549999) (end 152.131387 135.549999) (width 0.4) (layer F.Cu) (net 15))
 (segment (start 152.131387 135.549999) (end 153.899978 133.781408) (width 0.4) (layer F.Cu) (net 15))
 (segment (start 153.899978 133.781408) (end 153.899978 126.150022) (width 0.4) (layer F.Cu) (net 15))
 (segment (start 153.899978 126.150022) (end 154.66 125.39) (width 0.4) (layer F.Cu) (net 15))
 (segment (start 154.66 125.39) (end 156.66 125.39) (width 0.4) (layer F.Cu) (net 15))
 (segment (start 142.85 109.6) (end 144.05 109.6) (width 0.4) (layer F.Cu) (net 20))
 (segment (start 144.05 109.6) (end 146.29 111.84) (width 0.4) (layer F.Cu) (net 20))
 (segment (start 146.29 111.84) (end 146.568 111.84) (width 0.4) (layer F.Cu) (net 20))
 (segment (start 146.568 111.84) (end 148.6444 111.84) (width 0.4) (layer F.Cu) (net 20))
 (segment (start 142.85 111.6) (end 144.45 111.6) (width 0.4) (layer F.Cu) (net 21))
 (segment (start 146.568 113.11) (end 148.6444 113.11) (width 0.4) (layer F.Cu) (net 21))
 (segment (start 144.45 111.6) (end 145.96 113.11) (width 0.4) (layer F.Cu) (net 21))
 (segment (start 145.96 113.11) (end 146.568 113.11) (width 0.4) (layer F.Cu) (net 21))
 (segment (start 159.45 128.9) (end 159.45 131.25) (width 0.4) (layer F.Cu) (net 14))
 (segment (start 159.45 131.25) (end 159.15 131.55) (width 0.4) (layer F.Cu) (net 14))
 (segment (start 159.15 131.55) (end 155.518614 131.55) (width 0.4) (layer F.Cu) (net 14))
 (segment (start 155.518614 131.55) (end 154.699989 132.368625) (width 0.4) (layer F.Cu) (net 14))
 (segment (start 154.699989 132.368625) (end 154.699989 134.750011) (width 0.4) (layer F.Cu) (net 14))
 (segment (start 154.699989 134.750011) (end 152.8 136.65) (width 0.4) (layer F.Cu) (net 14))
 (segment (start 152.8 136.65) (end 152.8 136.725) (width 0.4) (layer F.Cu) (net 14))
 (segment (start 159.45 126.25) (end 159.45 121.2) (width 0.4) (layer F.Cu) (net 14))
 (segment (start 159.45 121.2) (end 158.56 120.31) (width 0.4) (layer F.Cu) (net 14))
 (segment (start 158.56 120.31) (end 156.66 120.31) (width 0.4) (layer F.Cu) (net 14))
 (segment (start 159.45 126.25) (end 159.45 128.9) (width 0.4) (layer F.Cu) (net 14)))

